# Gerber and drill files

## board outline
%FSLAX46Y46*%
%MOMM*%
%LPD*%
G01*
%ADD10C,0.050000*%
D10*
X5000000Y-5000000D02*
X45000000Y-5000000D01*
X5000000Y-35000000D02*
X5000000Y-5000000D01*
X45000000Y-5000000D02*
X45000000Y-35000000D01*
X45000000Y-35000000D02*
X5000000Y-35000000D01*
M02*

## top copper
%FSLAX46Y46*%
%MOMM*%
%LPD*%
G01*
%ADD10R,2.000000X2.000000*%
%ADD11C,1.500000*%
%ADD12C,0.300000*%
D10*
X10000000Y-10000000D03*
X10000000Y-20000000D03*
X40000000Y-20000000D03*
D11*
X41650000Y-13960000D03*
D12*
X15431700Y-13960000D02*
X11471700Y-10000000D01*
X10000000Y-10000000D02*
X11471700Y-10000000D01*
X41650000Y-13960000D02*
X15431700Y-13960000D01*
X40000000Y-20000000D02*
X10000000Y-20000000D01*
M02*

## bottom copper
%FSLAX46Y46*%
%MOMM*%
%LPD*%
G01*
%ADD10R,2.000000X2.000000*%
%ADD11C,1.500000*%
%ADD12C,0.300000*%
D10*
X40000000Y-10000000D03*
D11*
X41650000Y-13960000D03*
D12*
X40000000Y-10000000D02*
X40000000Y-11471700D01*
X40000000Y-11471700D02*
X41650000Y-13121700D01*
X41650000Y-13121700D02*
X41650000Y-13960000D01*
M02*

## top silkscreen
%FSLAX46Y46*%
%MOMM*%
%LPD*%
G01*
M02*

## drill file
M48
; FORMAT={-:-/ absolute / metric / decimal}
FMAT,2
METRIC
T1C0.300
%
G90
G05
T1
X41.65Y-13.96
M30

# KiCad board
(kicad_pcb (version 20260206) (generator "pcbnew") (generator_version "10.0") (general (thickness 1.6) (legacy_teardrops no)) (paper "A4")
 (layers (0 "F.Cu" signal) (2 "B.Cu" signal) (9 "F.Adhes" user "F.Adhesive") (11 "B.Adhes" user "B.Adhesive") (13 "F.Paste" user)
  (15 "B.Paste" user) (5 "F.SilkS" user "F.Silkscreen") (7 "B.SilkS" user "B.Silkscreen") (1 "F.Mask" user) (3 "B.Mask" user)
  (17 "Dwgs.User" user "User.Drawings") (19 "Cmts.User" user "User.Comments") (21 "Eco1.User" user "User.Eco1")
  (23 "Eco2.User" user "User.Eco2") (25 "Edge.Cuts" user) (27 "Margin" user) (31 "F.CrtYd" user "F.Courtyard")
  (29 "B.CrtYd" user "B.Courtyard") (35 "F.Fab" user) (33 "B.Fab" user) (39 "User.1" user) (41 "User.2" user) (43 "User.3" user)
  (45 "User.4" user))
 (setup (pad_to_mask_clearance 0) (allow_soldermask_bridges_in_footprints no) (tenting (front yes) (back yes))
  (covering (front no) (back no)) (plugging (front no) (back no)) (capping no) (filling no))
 (gr_line (start 5 5) (end 45 5) (stroke (width 0.05) (type default)) (layer "Edge.Cuts"))
 (gr_line (start 5 35) (end 5 5) (stroke (width 0.05) (type default)) (layer "Edge.Cuts"))
 (gr_line (start 45 5) (end 45 35) (stroke (width 0.05) (type default)) (layer "Edge.Cuts"))
 (gr_line (start 45 35) (end 5 35) (stroke (width 0.05) (type default)) (layer "Edge.Cuts"))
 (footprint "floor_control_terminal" (layer "F.Cu") (at 10 10)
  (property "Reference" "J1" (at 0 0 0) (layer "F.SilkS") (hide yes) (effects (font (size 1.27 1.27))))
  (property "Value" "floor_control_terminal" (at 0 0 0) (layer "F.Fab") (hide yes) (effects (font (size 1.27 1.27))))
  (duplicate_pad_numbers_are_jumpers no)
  (pad "1" smd rect (at 0 0) (size 2 2) (layers "F.Cu" "F.Paste" "F.Mask") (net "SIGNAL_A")))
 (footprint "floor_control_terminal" (layer "B.Cu") (at 40 10)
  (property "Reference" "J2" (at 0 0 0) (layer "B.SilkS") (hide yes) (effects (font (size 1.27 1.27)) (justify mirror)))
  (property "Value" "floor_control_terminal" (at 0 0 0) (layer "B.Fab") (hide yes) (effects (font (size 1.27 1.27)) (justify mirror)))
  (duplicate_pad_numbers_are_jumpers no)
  (pad "1" smd rect (at 0 0) (size 2 2) (layers "B.Cu" "B.Paste" "B.Mask") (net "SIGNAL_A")))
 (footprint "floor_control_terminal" (layer "F.Cu") (at 10 20)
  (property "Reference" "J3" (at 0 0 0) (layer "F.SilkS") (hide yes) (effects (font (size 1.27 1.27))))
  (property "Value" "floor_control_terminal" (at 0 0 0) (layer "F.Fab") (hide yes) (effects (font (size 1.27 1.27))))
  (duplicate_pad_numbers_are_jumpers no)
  (pad "1" smd rect (at 0 0) (size 2 2) (layers "F.Cu" "F.Paste" "F.Mask") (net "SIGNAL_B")))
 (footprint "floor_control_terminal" (layer "F.Cu") (at 40 20)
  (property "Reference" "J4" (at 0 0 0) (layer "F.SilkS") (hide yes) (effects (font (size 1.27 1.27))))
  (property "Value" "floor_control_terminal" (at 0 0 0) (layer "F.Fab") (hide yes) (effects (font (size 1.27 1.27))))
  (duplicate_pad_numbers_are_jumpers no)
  (pad "1" smd rect (at 0 0) (size 2 2) (layers "F.Cu" "F.Paste" "F.Mask") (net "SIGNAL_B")))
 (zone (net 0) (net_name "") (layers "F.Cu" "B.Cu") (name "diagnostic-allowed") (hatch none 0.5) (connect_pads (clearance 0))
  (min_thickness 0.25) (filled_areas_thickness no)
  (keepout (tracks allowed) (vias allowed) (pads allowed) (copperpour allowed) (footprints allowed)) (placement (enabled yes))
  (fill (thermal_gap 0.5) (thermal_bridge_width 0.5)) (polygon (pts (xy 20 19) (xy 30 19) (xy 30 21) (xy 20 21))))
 (segment (start 15.4317 13.96) (end 11.4717 10) (width 0.3) (layer "F.Cu") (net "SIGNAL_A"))
 (segment (start 10 10) (end 11.4717 10) (width 0.3) (layer "F.Cu") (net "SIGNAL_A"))
 (segment (start 41.65 13.96) (end 15.4317 13.96) (width 0.3) (layer "F.Cu") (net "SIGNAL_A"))
 (via (at 41.65 13.96) (size 1.5) (drill 0.3) (layers "F.Cu" "B.Cu") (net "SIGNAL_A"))
 (segment (start 40 10) (end 40 11.4717) (width 0.3) (layer "B.Cu") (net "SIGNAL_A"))
 (segment (start 40 11.4717) (end 41.65 13.1217) (width 0.3) (layer "B.Cu") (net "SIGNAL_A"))
 (segment (start 41.65 13.1217) (end 41.65 13.96) (width 0.3) (layer "B.Cu") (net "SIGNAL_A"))
 (segment (start 40 20) (end 10 20) (width 0.3) (layer "F.Cu") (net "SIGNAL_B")))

